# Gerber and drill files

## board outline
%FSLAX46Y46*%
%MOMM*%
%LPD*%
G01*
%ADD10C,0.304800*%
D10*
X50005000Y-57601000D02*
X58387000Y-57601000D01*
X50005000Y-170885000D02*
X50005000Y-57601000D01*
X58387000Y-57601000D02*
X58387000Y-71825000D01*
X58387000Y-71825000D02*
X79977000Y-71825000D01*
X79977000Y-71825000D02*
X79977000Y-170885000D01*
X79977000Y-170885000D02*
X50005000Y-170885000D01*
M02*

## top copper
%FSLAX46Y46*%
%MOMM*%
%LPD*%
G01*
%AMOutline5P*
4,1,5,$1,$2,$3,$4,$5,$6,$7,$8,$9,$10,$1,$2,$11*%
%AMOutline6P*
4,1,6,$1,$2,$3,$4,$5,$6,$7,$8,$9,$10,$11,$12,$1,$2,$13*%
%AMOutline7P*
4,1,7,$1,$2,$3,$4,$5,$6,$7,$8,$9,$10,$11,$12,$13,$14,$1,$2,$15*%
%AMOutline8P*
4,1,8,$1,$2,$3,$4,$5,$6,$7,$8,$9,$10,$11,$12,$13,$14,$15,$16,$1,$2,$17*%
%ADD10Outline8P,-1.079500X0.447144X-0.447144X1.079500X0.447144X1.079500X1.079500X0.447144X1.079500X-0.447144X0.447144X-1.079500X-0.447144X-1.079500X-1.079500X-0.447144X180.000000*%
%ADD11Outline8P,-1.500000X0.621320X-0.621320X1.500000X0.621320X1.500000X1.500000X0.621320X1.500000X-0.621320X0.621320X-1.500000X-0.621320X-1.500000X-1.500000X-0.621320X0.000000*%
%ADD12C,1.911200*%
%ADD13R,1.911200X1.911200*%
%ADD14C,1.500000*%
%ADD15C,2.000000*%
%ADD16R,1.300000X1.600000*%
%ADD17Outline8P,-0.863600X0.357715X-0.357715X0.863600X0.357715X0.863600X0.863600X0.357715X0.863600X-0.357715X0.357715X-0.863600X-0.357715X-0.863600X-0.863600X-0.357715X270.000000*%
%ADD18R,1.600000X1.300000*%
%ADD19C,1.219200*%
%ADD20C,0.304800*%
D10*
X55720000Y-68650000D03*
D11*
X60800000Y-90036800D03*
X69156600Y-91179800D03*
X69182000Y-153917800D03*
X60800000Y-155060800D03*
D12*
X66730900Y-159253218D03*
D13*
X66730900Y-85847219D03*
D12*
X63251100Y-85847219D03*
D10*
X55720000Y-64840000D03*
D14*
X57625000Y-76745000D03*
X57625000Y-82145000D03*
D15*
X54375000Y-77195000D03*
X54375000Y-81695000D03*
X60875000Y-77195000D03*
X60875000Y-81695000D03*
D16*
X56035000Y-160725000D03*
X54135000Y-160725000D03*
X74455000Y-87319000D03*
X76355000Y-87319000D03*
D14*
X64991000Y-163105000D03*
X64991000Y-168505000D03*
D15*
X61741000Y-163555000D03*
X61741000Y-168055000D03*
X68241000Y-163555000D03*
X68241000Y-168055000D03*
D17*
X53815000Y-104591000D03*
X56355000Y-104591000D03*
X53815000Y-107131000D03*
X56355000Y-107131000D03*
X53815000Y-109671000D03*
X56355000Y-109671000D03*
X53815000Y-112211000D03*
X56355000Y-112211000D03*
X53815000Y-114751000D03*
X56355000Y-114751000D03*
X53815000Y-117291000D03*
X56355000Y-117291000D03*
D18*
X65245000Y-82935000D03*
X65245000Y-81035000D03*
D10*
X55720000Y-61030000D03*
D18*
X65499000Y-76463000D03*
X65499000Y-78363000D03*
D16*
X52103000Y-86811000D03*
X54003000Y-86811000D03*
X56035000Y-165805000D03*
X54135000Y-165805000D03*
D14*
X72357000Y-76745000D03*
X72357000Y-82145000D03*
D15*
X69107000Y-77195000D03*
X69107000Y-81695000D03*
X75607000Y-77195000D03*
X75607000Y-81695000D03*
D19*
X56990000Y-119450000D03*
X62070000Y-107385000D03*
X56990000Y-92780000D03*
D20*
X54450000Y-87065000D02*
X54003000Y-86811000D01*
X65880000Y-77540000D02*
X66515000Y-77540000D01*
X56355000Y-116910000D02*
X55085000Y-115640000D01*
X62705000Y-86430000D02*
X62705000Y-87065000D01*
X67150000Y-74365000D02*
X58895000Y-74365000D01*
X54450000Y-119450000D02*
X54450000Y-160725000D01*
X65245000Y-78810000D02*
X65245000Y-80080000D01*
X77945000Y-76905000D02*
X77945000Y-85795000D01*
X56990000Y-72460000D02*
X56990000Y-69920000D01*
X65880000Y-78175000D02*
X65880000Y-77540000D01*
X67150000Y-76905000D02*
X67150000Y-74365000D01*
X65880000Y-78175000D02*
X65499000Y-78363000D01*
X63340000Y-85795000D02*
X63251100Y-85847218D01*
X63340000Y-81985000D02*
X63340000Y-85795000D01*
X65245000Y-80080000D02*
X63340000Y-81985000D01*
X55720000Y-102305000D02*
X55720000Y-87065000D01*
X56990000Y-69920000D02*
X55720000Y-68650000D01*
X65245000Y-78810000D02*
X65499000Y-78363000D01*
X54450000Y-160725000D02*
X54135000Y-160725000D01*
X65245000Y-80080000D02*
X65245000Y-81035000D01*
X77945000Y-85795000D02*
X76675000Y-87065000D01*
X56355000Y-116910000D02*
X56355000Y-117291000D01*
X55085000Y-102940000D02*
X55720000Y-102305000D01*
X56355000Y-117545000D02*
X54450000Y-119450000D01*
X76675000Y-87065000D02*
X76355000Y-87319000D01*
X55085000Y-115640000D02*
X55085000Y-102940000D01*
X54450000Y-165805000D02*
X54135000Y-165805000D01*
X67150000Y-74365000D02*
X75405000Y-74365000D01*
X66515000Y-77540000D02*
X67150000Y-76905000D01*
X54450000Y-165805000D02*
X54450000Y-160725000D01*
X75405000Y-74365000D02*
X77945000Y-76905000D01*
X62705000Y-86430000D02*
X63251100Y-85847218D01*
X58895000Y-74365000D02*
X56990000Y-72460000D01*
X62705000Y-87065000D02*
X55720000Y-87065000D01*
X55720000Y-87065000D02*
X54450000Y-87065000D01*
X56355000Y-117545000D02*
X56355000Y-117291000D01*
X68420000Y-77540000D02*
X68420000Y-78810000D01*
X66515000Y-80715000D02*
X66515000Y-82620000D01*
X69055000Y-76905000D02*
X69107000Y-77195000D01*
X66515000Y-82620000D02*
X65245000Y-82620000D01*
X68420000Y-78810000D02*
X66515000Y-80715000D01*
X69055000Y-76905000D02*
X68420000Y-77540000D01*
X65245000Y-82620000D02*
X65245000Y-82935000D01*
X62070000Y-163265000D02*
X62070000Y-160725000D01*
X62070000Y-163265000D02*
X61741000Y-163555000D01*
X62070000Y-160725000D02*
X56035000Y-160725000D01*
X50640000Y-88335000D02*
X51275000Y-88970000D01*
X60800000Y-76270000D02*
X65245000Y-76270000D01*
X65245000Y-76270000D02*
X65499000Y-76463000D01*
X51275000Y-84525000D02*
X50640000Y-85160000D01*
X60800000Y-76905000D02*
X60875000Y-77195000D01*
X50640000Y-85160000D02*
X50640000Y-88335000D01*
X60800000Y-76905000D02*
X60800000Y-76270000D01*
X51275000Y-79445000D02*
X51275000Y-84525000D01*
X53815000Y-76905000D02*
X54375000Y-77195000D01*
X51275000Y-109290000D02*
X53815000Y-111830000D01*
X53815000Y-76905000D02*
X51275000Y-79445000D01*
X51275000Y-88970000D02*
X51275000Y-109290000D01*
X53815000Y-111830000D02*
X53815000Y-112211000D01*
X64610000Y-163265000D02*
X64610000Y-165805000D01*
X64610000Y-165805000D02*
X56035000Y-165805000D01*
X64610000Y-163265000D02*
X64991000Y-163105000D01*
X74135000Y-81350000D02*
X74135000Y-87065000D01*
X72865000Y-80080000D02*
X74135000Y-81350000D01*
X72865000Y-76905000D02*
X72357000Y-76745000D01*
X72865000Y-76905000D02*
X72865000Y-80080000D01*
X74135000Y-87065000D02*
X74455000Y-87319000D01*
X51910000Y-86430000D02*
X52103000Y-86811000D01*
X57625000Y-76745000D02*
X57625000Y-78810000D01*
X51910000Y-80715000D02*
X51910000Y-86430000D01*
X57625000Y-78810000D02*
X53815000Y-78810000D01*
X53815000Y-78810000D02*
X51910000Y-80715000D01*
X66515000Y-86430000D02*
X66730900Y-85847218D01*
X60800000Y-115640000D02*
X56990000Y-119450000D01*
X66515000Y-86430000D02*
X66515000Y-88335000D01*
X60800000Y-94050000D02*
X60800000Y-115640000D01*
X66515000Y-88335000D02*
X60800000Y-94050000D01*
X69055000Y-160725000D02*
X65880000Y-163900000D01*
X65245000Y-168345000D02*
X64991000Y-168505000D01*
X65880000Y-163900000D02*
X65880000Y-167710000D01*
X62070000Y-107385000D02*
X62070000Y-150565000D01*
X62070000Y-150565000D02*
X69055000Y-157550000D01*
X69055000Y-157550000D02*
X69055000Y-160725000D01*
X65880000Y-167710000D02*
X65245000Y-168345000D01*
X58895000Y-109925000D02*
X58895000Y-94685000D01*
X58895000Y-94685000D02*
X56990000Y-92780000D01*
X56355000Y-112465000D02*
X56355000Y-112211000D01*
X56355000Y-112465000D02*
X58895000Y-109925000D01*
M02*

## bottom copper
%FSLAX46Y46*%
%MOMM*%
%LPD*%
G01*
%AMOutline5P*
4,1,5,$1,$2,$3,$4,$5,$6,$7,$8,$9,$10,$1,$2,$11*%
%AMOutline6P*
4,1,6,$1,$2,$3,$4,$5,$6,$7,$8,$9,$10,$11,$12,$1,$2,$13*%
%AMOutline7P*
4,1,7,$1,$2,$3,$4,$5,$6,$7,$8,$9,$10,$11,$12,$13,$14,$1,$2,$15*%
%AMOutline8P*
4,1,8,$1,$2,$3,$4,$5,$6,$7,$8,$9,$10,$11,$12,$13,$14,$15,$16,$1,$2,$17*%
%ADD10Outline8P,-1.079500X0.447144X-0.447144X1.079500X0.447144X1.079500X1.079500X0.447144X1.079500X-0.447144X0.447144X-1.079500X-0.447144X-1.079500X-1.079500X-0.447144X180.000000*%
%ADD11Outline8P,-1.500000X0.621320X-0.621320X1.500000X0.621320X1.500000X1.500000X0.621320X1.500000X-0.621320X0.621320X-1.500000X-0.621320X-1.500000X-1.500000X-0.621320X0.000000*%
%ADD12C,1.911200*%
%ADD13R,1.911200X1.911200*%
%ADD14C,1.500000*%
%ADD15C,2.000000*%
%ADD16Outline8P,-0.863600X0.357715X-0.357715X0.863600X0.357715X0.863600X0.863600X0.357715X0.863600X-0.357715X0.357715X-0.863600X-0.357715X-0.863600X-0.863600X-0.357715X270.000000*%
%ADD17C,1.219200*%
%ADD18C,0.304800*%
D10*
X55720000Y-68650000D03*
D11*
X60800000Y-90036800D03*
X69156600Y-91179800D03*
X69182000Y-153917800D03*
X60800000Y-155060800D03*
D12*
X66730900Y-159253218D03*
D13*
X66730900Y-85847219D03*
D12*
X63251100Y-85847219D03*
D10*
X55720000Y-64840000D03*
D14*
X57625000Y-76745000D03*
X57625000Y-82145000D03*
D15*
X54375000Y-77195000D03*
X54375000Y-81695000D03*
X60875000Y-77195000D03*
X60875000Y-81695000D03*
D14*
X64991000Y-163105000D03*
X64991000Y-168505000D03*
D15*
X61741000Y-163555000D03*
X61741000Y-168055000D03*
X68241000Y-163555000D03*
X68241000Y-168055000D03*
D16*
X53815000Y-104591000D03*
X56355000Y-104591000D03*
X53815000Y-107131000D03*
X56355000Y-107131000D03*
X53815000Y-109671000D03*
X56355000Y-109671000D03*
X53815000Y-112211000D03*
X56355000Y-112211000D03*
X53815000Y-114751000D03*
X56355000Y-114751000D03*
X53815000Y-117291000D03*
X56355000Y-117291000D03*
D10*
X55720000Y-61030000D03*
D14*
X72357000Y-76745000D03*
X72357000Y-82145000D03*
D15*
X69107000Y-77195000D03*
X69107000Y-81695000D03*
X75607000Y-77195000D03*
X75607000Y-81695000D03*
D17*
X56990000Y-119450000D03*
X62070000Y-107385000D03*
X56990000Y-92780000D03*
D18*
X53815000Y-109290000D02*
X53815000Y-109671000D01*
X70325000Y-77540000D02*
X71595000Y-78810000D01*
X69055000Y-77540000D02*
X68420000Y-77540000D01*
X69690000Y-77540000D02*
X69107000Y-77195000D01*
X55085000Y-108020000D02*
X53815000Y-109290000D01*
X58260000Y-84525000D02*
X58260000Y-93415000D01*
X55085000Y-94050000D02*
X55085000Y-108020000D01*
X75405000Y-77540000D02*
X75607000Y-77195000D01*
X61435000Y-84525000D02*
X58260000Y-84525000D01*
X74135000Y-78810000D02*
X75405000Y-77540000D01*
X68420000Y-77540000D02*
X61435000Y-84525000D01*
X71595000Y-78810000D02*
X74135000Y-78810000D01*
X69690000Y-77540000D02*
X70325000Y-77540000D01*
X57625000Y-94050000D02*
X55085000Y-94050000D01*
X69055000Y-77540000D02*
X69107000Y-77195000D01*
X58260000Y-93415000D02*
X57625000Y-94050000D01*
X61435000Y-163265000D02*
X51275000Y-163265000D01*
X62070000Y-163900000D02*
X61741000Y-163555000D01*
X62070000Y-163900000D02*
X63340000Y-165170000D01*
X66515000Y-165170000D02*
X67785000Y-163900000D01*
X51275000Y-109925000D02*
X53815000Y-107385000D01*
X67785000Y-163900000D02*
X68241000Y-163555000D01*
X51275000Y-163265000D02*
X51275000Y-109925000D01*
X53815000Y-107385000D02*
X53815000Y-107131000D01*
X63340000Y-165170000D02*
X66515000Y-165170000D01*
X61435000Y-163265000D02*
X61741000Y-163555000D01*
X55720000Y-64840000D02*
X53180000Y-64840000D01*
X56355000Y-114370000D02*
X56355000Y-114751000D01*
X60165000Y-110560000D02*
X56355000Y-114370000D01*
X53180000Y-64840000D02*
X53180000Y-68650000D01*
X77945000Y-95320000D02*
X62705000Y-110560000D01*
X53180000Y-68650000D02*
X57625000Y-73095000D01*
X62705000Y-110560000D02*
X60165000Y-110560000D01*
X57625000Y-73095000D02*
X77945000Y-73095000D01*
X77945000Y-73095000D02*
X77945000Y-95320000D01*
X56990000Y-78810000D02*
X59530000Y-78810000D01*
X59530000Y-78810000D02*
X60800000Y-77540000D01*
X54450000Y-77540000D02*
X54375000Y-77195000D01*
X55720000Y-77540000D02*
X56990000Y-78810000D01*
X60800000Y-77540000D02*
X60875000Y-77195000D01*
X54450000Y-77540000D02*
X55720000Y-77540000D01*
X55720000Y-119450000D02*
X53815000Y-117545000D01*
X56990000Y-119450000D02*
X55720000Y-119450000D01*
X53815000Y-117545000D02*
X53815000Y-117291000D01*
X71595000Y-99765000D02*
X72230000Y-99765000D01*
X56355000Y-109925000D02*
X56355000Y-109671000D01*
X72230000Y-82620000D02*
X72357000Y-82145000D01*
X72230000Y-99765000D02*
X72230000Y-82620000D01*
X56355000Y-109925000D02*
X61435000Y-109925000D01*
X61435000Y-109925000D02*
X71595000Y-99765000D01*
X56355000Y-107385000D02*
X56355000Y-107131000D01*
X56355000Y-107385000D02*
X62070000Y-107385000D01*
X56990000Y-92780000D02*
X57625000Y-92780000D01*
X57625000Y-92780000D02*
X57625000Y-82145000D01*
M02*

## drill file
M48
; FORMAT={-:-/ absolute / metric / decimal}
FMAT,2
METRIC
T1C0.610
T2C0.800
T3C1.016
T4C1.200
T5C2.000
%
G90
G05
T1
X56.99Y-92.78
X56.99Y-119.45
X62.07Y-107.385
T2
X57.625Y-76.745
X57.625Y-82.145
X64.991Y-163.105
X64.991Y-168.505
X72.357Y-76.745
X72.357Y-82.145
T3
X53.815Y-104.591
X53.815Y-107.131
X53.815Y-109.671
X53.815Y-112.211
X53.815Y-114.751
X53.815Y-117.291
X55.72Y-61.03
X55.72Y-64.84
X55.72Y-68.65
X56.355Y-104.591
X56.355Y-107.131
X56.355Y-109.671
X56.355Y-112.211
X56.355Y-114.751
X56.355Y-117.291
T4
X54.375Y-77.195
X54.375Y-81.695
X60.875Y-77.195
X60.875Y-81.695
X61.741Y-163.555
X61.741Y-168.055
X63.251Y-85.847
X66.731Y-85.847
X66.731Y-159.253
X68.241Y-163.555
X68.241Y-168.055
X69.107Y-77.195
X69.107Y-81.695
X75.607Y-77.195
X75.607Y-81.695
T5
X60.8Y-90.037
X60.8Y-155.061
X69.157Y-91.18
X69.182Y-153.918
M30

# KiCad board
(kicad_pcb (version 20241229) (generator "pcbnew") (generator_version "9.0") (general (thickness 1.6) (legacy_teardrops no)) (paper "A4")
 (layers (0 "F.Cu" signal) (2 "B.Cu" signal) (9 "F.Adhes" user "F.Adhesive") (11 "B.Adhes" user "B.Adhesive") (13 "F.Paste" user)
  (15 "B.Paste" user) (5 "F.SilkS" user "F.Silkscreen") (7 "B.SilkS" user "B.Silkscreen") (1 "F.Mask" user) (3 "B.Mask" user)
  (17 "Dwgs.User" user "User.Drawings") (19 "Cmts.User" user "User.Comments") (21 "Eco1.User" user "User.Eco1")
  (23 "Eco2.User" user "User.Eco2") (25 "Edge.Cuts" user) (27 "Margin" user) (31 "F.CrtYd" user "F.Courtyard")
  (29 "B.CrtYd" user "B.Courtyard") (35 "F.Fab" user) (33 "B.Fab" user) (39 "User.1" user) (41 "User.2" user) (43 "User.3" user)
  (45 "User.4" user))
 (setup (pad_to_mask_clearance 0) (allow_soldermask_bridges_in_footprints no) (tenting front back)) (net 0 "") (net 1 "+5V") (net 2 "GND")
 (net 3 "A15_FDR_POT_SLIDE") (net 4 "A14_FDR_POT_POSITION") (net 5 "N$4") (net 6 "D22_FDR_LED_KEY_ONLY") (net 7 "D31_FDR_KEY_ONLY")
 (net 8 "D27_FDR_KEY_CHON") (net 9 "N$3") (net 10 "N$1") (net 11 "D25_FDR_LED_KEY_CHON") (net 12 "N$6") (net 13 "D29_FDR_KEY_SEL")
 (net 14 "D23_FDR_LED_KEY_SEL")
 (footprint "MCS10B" (layer "F.Cu") (at 55.72 68.65 180)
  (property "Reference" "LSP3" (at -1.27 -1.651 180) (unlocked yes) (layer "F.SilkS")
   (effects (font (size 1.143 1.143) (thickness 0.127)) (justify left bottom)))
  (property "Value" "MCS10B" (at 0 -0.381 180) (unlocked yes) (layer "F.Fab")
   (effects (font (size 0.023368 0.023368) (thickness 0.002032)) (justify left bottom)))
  (pad "MP" thru_hole roundrect (at 0 0 180) (size 2.159 2.159) (drill 1.016) (layers "*.Cu" "*.Mask") (remove_unused_layers no)
   (roundrect_rratio 0.25) (chamfer_ratio 0.2928932188) (chamfer top_left top_right bottom_left bottom_right) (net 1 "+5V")
   (solder_mask_margin 0.1016) (thermal_bridge_angle 0)))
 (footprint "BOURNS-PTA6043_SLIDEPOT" (layer "F.Cu") (at 64.991 116.529)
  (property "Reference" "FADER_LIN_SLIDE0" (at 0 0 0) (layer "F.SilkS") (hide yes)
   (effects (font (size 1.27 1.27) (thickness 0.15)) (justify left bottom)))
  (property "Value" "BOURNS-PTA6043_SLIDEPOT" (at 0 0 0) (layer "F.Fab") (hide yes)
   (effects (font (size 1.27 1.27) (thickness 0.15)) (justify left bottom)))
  (pad "MOUNT1" thru_hole roundrect (at -4.191 -26.4922) (size 3 3) (drill 2) (layers "*.Cu" "*.Mask") (remove_unused_layers no)
   (roundrect_rratio 0.25) (chamfer_ratio 0.2928932188) (chamfer top_left top_right bottom_left bottom_right) (solder_mask_margin 0.1016)
   (thermal_bridge_angle 0))
  (pad "MOUNT2" thru_hole roundrect (at 4.1656 -25.3492) (size 3 3) (drill 2) (layers "*.Cu" "*.Mask") (remove_unused_layers no)
   (roundrect_rratio 0.25) (chamfer_ratio 0.2928932188) (chamfer top_left top_right bottom_left bottom_right) (solder_mask_margin 0.1016)
   (thermal_bridge_angle 0))
  (pad "MOUNT3" thru_hole roundrect (at 4.191 37.3888) (size 3 3) (drill 2) (layers "*.Cu" "*.Mask") (remove_unused_layers no)
   (roundrect_rratio 0.25) (chamfer_ratio 0.2928932188) (chamfer top_left top_right bottom_left bottom_right) (solder_mask_margin 0.1016)
   (thermal_bridge_angle 0))
  (pad "MOUNT4" thru_hole roundrect (at -4.191 38.5318) (size 3 3) (drill 2) (layers "*.Cu" "*.Mask") (remove_unused_layers no)
   (roundrect_rratio 0.25) (chamfer_ratio 0.2928932188) (chamfer top_left top_right bottom_left bottom_right) (solder_mask_margin 0.1016)
   (thermal_bridge_angle 0))
  (pad "P$1" thru_hole circle (at 1.7399 42.724218) (size 1.9112 1.9112) (drill 1.2) (layers "*.Cu" "*.Mask") (remove_unused_layers no)
   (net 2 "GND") (solder_mask_margin 0.1016) (thermal_bridge_angle 0))
  (pad "P$2" thru_hole rect (at 1.7399 -30.681781) (size 1.9112 1.9112) (drill 1.2) (layers "*.Cu" "*.Mask") (remove_unused_layers no)
   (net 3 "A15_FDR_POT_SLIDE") (solder_mask_margin 0.1016) (thermal_bridge_angle 0))
  (pad "P$3" thru_hole circle (at -1.7399 -30.681781) (size 1.9112 1.9112) (drill 1.2) (layers "*.Cu" "*.Mask") (remove_unused_layers no)
   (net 1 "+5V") (solder_mask_margin 0.1016) (thermal_bridge_angle 0)))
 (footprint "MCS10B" (layer "F.Cu") (at 55.72 64.84 180)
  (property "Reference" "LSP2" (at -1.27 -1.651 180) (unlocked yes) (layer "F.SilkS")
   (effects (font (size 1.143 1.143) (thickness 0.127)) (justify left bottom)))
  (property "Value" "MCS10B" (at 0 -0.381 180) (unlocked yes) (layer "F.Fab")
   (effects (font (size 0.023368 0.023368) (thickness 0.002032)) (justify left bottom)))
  (pad "MP" thru_hole roundrect (at 0 0 180) (size 2.159 2.159) (drill 1.016) (layers "*.Cu" "*.Mask") (remove_unused_layers no)
   (roundrect_rratio 0.25) (chamfer_ratio 0.2928932188) (chamfer top_left top_right bottom_left bottom_right) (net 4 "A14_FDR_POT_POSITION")
   (solder_mask_margin 0.1016) (thermal_bridge_angle 0)))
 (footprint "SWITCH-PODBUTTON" (layer "F.Cu") (at 57.625 79.445)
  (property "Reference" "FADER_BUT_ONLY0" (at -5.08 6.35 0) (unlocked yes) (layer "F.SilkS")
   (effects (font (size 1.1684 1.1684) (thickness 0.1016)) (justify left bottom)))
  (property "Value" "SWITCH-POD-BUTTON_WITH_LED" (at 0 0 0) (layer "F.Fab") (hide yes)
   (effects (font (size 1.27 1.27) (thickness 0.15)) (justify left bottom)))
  (pad "LEDA" thru_hole circle (at 0 -2.7) (size 1.5 1.5) (drill 0.8) (layers "*.Cu" "*.Mask") (remove_unused_layers no) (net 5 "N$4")
   (solder_mask_margin 0.1016) (thermal_bridge_angle 0))
  (pad "LEDB" thru_hole circle (at 0 2.7) (size 1.5 1.5) (drill 0.8) (layers "*.Cu" "*.Mask") (remove_unused_layers no)
   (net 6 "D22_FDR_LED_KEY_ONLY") (solder_mask_margin 0.1016) (thermal_bridge_angle 0))
  (pad "SW1A" thru_hole circle (at -3.25 -2.25) (size 2 2) (drill 1.2) (layers "*.Cu" "*.Mask") (remove_unused_layers no)
   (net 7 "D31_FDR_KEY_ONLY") (solder_mask_margin 0.1016) (thermal_bridge_angle 0))
  (pad "SW1B" thru_hole circle (at -3.25 2.25) (size 2 2) (drill 1.2) (layers "*.Cu" "*.Mask") (remove_unused_layers no) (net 2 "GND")
   (solder_mask_margin 0.1016) (thermal_bridge_angle 0))
  (pad "SW2A" thru_hole circle (at 3.25 -2.25) (size 2 2) (drill 1.2) (layers "*.Cu" "*.Mask") (remove_unused_layers no)
   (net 7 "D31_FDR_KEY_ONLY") (solder_mask_margin 0.1016) (thermal_bridge_angle 0))
  (pad "SW2B" thru_hole circle (at 3.25 2.25) (size 2 2) (drill 1.2) (layers "*.Cu" "*.Mask") (remove_unused_layers no) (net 2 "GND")
   (solder_mask_margin 0.1016) (thermal_bridge_angle 0)))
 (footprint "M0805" (layer "F.Cu") (at 55.085 160.725 180)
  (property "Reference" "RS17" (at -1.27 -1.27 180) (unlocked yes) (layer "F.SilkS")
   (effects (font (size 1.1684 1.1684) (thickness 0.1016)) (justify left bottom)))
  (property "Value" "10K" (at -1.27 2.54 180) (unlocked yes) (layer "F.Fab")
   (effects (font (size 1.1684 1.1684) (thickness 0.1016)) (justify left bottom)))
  (pad "1" smd rect (at -0.95 0 180) (size 1.3 1.6) (layers "F.Cu" "F.Mask" "F.Paste") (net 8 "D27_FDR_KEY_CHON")
   (solder_mask_margin 0.1016) (solder_paste_margin 0) (thermal_bridge_angle 0))
  (pad "2" smd rect (at 0.95 0 180) (size 1.3 1.6) (layers "F.Cu" "F.Mask" "F.Paste") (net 1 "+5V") (solder_mask_margin 0.1016)
   (solder_paste_margin 0) (thermal_bridge_angle 0)))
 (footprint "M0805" (layer "F.Cu") (at 75.405 87.319)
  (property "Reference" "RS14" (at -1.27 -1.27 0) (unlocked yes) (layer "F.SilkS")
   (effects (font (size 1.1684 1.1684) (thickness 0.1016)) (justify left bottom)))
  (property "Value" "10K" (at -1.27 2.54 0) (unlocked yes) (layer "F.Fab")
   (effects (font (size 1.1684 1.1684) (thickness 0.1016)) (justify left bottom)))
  (pad "1" smd rect (at -0.95 0) (size 1.3 1.6) (layers "F.Cu" "F.Mask" "F.Paste") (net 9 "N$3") (solder_mask_margin 0.1016)
   (solder_paste_margin 0) (thermal_bridge_angle 0))
  (pad "2" smd rect (at 0.95 0) (size 1.3 1.6) (layers "F.Cu" "F.Mask" "F.Paste") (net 1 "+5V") (solder_mask_margin 0.1016)
   (solder_paste_margin 0) (thermal_bridge_angle 0)))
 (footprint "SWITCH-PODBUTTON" (layer "F.Cu") (at 64.991 165.805)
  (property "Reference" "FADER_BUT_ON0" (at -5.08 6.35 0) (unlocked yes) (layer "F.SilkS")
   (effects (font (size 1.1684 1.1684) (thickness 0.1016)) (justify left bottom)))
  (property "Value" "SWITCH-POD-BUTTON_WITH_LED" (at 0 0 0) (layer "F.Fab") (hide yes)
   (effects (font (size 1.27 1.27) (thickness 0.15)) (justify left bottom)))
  (pad "LEDA" thru_hole circle (at 0 -2.7) (size 1.5 1.5) (drill 0.8) (layers "*.Cu" "*.Mask") (remove_unused_layers no) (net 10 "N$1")
   (solder_mask_margin 0.1016) (thermal_bridge_angle 0))
  (pad "LEDB" thru_hole circle (at 0 2.7) (size 1.5 1.5) (drill 0.8) (layers "*.Cu" "*.Mask") (remove_unused_layers no)
   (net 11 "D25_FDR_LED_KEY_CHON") (solder_mask_margin 0.1016) (thermal_bridge_angle 0))
  (pad "SW1A" thru_hole circle (at -3.25 -2.25) (size 2 2) (drill 1.2) (layers "*.Cu" "*.Mask") (remove_unused_layers no)
   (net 8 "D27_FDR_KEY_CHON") (solder_mask_margin 0.1016) (thermal_bridge_angle 0))
  (pad "SW1B" thru_hole circle (at -3.25 2.25) (size 2 2) (drill 1.2) (layers "*.Cu" "*.Mask") (remove_unused_layers no) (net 2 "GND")
   (solder_mask_margin 0.1016) (thermal_bridge_angle 0))
  (pad "SW2A" thru_hole circle (at 3.25 -2.25) (size 2 2) (drill 1.2) (layers "*.Cu" "*.Mask") (remove_unused_layers no)
   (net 8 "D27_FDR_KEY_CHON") (solder_mask_margin 0.1016) (thermal_bridge_angle 0))
  (pad "SW2B" thru_hole circle (at 3.25 2.25) (size 2 2) (drill 1.2) (layers "*.Cu" "*.Mask") (remove_unused_layers no) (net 2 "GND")
   (solder_mask_margin 0.1016) (thermal_bridge_angle 0)))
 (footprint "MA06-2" (layer "F.Cu") (at 55.085 110.941 -90)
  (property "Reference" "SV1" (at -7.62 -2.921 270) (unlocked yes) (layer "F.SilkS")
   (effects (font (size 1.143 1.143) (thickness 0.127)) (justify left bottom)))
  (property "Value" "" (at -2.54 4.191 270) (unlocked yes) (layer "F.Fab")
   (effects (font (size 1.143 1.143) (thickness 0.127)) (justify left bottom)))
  (pad "1" thru_hole roundrect (at -6.35 1.27 270) (size 1.7272 1.7272) (drill 1.016) (layers "*.Cu" "*.Mask") (remove_unused_layers no)
   (roundrect_rratio 0.25) (chamfer_ratio 0.2928932188) (chamfer top_left top_right bottom_left bottom_right) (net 2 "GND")
   (solder_mask_margin 0.1016) (thermal_bridge_angle 0))
  (pad "2" thru_hole roundrect (at -6.35 -1.27 270) (size 1.7272 1.7272) (drill 1.016) (layers "*.Cu" "*.Mask") (remove_unused_layers no)
   (roundrect_rratio 0.25) (chamfer_ratio 0.2928932188) (chamfer top_left top_right bottom_left bottom_right) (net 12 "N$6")
   (solder_mask_margin 0.1016) (thermal_bridge_angle 0))
  (pad "3" thru_hole roundrect (at -3.81 1.27 270) (size 1.7272 1.7272) (drill 1.016) (layers "*.Cu" "*.Mask") (remove_unused_layers no)
   (roundrect_rratio 0.25) (chamfer_ratio 0.2928932188) (chamfer top_left top_right bottom_left bottom_right) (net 8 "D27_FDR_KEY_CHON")
   (solder_mask_margin 0.1016) (thermal_bridge_angle 0))
  (pad "4" thru_hole roundrect (at -3.81 -1.27 270) (size 1.7272 1.7272) (drill 1.016) (layers "*.Cu" "*.Mask") (remove_unused_layers no)
   (roundrect_rratio 0.25) (chamfer_ratio 0.2928932188) (chamfer top_left top_right bottom_left bottom_right)
   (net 11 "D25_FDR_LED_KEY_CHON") (solder_mask_margin 0.1016) (thermal_bridge_angle 0))
  (pad "5" thru_hole roundrect (at -1.27 1.27 270) (size 1.7272 1.7272) (drill 1.016) (layers "*.Cu" "*.Mask") (remove_unused_layers no)
   (roundrect_rratio 0.25) (chamfer_ratio 0.2928932188) (chamfer top_left top_right bottom_left bottom_right) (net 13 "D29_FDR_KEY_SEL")
   (solder_mask_margin 0.1016) (thermal_bridge_angle 0))
  (pad "6" thru_hole roundrect (at -1.27 -1.27 270) (size 1.7272 1.7272) (drill 1.016) (layers "*.Cu" "*.Mask") (remove_unused_layers no)
   (roundrect_rratio 0.25) (chamfer_ratio 0.2928932188) (chamfer top_left top_right bottom_left bottom_right) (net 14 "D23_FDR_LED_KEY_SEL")
   (solder_mask_margin 0.1016) (thermal_bridge_angle 0))
  (pad "7" thru_hole roundrect (at 1.27 1.27 270) (size 1.7272 1.7272) (drill 1.016) (layers "*.Cu" "*.Mask") (remove_unused_layers no)
   (roundrect_rratio 0.25) (chamfer_ratio 0.2928932188) (chamfer top_left top_right bottom_left bottom_right) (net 7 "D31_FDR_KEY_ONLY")
   (solder_mask_margin 0.1016) (thermal_bridge_angle 0))
  (pad "8" thru_hole roundrect (at 1.27 -1.27 270) (size 1.7272 1.7272) (drill 1.016) (layers "*.Cu" "*.Mask") (remove_unused_layers no)
   (roundrect_rratio 0.25) (chamfer_ratio 0.2928932188) (chamfer top_left top_right bottom_left bottom_right) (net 6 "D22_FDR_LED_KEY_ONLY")
   (solder_mask_margin 0.1016) (thermal_bridge_angle 0))
  (pad "9" thru_hole roundrect (at 3.81 1.27 270) (size 1.7272 1.7272) (drill 1.016) (layers "*.Cu" "*.Mask") (remove_unused_layers no)
   (roundrect_rratio 0.25) (chamfer_ratio 0.2928932188) (chamfer top_left top_right bottom_left bottom_right) (solder_mask_margin 0.1016)
   (thermal_bridge_angle 0))
  (pad "10" thru_hole roundrect (at 3.81 -1.27 270) (size 1.7272 1.7272) (drill 1.016) (layers "*.Cu" "*.Mask") (remove_unused_layers no)
   (roundrect_rratio 0.25) (chamfer_ratio 0.2928932188) (chamfer top_left top_right bottom_left bottom_right) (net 4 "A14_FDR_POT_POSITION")
   (solder_mask_margin 0.1016) (thermal_bridge_angle 0))
  (pad "11" thru_hole roundrect (at 6.35 1.27 270) (size 1.7272 1.7272) (drill 1.016) (layers "*.Cu" "*.Mask") (remove_unused_layers no)
   (roundrect_rratio 0.25) (chamfer_ratio 0.2928932188) (chamfer top_left top_right bottom_left bottom_right) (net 3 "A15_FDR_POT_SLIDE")
   (solder_mask_margin 0.1016) (thermal_bridge_angle 0))
  (pad "12" thru_hole roundrect (at 6.35 -1.27 270) (size 1.7272 1.7272) (drill 1.016) (layers "*.Cu" "*.Mask") (remove_unused_layers no)
   (roundrect_rratio 0.25) (chamfer_ratio 0.2928932188) (chamfer top_left top_right bottom_left bottom_right) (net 1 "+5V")
   (solder_mask_margin 0.1016) (thermal_bridge_angle 0)))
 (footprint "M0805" (layer "F.Cu") (at 65.245 81.985 90)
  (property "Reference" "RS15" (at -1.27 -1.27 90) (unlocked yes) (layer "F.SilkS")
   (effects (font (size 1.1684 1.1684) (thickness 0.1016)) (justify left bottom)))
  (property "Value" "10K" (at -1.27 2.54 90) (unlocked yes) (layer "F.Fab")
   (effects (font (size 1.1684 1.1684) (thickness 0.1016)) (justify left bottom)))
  (pad "1" smd rect (at -0.95 0 90) (size 1.3 1.6) (layers "F.Cu" "F.Mask" "F.Paste") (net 13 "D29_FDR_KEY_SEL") (solder_mask_margin 0.1016)
   (solder_paste_margin 0) (thermal_bridge_angle 0))
  (pad "2" smd rect (at 0.95 0 90) (size 1.3 1.6) (layers "F.Cu" "F.Mask" "F.Paste") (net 1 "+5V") (solder_mask_margin 0.1016)
   (solder_paste_margin 0) (thermal_bridge_angle 0)))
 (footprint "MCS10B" (layer "F.Cu") (at 55.72 61.03 180)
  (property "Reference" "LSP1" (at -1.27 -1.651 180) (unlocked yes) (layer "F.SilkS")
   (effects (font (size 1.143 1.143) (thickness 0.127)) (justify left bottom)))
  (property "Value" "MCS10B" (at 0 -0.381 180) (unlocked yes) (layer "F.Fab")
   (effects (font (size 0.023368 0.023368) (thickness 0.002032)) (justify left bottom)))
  (pad "MP" thru_hole roundrect (at 0 0 180) (size 2.159 2.159) (drill 1.016) (layers "*.Cu" "*.Mask") (remove_unused_layers no)
   (roundrect_rratio 0.25) (chamfer_ratio 0.2928932188) (chamfer top_left top_right bottom_left bottom_right) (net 2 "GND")
   (solder_mask_margin 0.1016) (thermal_bridge_angle 0)))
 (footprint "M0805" (layer "F.Cu") (at 65.499 77.413 -90)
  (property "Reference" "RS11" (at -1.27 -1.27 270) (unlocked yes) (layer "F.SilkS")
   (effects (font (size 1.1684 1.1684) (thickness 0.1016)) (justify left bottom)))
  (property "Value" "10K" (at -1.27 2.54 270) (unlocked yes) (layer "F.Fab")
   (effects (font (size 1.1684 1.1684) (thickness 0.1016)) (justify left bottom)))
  (pad "1" smd rect (at -0.95 0 270) (size 1.3 1.6) (layers "F.Cu" "F.Mask" "F.Paste") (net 7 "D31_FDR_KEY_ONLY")
   (solder_mask_margin 0.1016) (solder_paste_margin 0) (thermal_bridge_angle 0))
  (pad "2" smd rect (at 0.95 0 270) (size 1.3 1.6) (layers "F.Cu" "F.Mask" "F.Paste") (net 1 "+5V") (solder_mask_margin 0.1016)
   (solder_paste_margin 0) (thermal_bridge_angle 0)))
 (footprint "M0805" (layer "F.Cu") (at 53.053 86.811)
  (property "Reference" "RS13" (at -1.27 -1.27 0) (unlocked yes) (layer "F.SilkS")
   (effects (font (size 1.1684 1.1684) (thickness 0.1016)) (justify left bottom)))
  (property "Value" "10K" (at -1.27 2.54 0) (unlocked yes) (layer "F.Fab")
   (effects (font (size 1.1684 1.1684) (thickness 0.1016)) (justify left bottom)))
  (pad "1" smd rect (at -0.95 0) (size 1.3 1.6) (layers "F.Cu" "F.Mask" "F.Paste") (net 5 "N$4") (solder_mask_margin 0.1016)
   (solder_paste_margin 0) (thermal_bridge_angle 0))
  (pad "2" smd rect (at 0.95 0) (size 1.3 1.6) (layers "F.Cu" "F.Mask" "F.Paste") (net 1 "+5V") (solder_mask_margin 0.1016)
   (solder_paste_margin 0) (thermal_bridge_angle 0)))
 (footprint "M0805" (layer "F.Cu") (at 55.085 165.805 180)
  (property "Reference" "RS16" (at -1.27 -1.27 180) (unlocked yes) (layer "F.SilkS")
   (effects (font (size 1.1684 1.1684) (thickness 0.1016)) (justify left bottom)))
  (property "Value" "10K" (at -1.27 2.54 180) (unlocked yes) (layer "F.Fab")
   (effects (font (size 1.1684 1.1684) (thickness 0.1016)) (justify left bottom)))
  (pad "1" smd rect (at -0.95 0 180) (size 1.3 1.6) (layers "F.Cu" "F.Mask" "F.Paste") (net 10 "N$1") (solder_mask_margin 0.1016)
   (solder_paste_margin 0) (thermal_bridge_angle 0))
  (pad "2" smd rect (at 0.95 0 180) (size 1.3 1.6) (layers "F.Cu" "F.Mask" "F.Paste") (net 1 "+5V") (solder_mask_margin 0.1016)
   (solder_paste_margin 0) (thermal_bridge_angle 0)))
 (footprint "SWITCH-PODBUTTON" (layer "F.Cu") (at 72.357 79.445)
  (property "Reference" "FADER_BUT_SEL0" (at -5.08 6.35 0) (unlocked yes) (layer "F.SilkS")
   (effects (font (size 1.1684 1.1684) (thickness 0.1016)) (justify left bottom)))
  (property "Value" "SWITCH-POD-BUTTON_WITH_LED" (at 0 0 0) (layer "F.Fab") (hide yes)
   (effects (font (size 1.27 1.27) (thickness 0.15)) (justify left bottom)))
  (pad "LEDA" thru_hole circle (at 0 -2.7) (size 1.5 1.5) (drill 0.8) (layers "*.Cu" "*.Mask") (remove_unused_layers no) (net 9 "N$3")
   (solder_mask_margin 0.1016) (thermal_bridge_angle 0))
  (pad "LEDB" thru_hole circle (at 0 2.7) (size 1.5 1.5) (drill 0.8) (layers "*.Cu" "*.Mask") (remove_unused_layers no)
   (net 14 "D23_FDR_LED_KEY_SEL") (solder_mask_margin 0.1016) (thermal_bridge_angle 0))
  (pad "SW1A" thru_hole circle (at -3.25 -2.25) (size 2 2) (drill 1.2) (layers "*.Cu" "*.Mask") (remove_unused_layers no)
   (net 13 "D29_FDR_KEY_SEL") (solder_mask_margin 0.1016) (thermal_bridge_angle 0))
  (pad "SW1B" thru_hole circle (at -3.25 2.25) (size 2 2) (drill 1.2) (layers "*.Cu" "*.Mask") (remove_unused_layers no) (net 2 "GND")
   (solder_mask_margin 0.1016) (thermal_bridge_angle 0))
  (pad "SW2A" thru_hole circle (at 3.25 -2.25) (size 2 2) (drill 1.2) (layers "*.Cu" "*.Mask") (remove_unused_layers no)
   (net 13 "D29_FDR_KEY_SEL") (solder_mask_margin 0.1016) (thermal_bridge_angle 0))
  (pad "SW2B" thru_hole circle (at 3.25 2.25) (size 2 2) (drill 1.2) (layers "*.Cu" "*.Mask") (remove_unused_layers no) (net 2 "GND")
   (solder_mask_margin 0.1016) (thermal_bridge_angle 0)))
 (gr_line (start 50.005 57.601) (end 58.387 57.601) (stroke (width 0.3048) (type solid)) (layer "Edge.Cuts"))
 (gr_line (start 50.005 170.885) (end 50.005 57.601) (stroke (width 0.3048) (type solid)) (layer "Edge.Cuts"))
 (gr_line (start 58.387 57.601) (end 58.387 71.825) (stroke (width 0.3048) (type solid)) (layer "Edge.Cuts"))
 (gr_line (start 58.387 71.825) (end 79.977 71.825) (stroke (width 0.3048) (type solid)) (layer "Edge.Cuts"))
 (gr_line (start 79.977 71.825) (end 79.977 170.885) (stroke (width 0.3048) (type solid)) (layer "Edge.Cuts"))
 (gr_line (start 79.977 170.885) (end 50.005 170.885) (stroke (width 0.3048) (type solid)) (layer "Edge.Cuts"))
 (segment (start 54.45 87.065) (end 54.003 86.811) (width 0.3048) (layer "F.Cu") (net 1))
 (segment (start 65.88 77.54) (end 66.515 77.54) (width 0.3048) (layer "F.Cu") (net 1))
 (segment (start 56.355 116.91) (end 55.085 115.64) (width 0.3048) (layer "F.Cu") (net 1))
 (segment (start 62.705 86.43) (end 62.705 87.065) (width 0.3048) (layer "F.Cu") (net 1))
 (segment (start 67.15 74.365) (end 58.895 74.365) (width 0.3048) (layer "F.Cu") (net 1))
 (segment (start 54.45 119.45) (end 54.45 160.725) (width 0.3048) (layer "F.Cu") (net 1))
 (segment (start 65.245 78.81) (end 65.245 80.08) (width 0.3048) (layer "F.Cu") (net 1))
 (segment (start 77.945 76.905) (end 77.945 85.795) (width 0.3048) (layer "F.Cu") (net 1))
 (segment (start 56.99 72.46) (end 56.99 69.92) (width 0.3048) (layer "F.Cu") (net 1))
 (segment (start 65.88 78.175) (end 65.88 77.54) (width 0.3048) (layer "F.Cu") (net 1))
 (segment (start 67.15 76.905) (end 67.15 74.365) (width 0.3048) (layer "F.Cu") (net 1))
 (segment (start 65.88 78.175) (end 65.499 78.363) (width 0.3048) (layer "F.Cu") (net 1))
 (segment (start 63.34 85.795) (end 63.2511 85.847218) (width 0.3048) (layer "F.Cu") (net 1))
 (segment (start 63.34 81.985) (end 63.34 85.795) (width 0.3048) (layer "F.Cu") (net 1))
 (segment (start 65.245 80.08) (end 63.34 81.985) (width 0.3048) (layer "F.Cu") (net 1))
 (segment (start 55.72 102.305) (end 55.72 87.065) (width 0.3048) (layer "F.Cu") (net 1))
 (segment (start 56.99 69.92) (end 55.72 68.65) (width 0.3048) (layer "F.Cu") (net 1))
 (segment (start 65.245 78.81) (end 65.499 78.363) (width 0.3048) (layer "F.Cu") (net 1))
 (segment (start 54.45 160.725) (end 54.135 160.725) (width 0.3048) (layer "F.Cu") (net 1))
 (segment (start 65.245 80.08) (end 65.245 81.035) (width 0.3048) (layer "F.Cu") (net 1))
 (segment (start 77.945 85.795) (end 76.675 87.065) (width 0.3048) (layer "F.Cu") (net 1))
 (segment (start 56.355 116.91) (end 56.355 117.291) (width 0.3048) (layer "F.Cu") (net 1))
 (segment (start 55.085 102.94) (end 55.72 102.305) (width 0.3048) (layer "F.Cu") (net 1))
 (segment (start 56.355 117.545) (end 54.45 119.45) (width 0.3048) (layer "F.Cu") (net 1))
 (segment (start 76.675 87.065) (end 76.355 87.319) (width 0.3048) (layer "F.Cu") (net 1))
 (segment (start 55.085 115.64) (end 55.085 102.94) (width 0.3048) (layer "F.Cu") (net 1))
 (segment (start 54.45 165.805) (end 54.135 165.805) (width 0.3048) (layer "F.Cu") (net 1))
 (segment (start 67.15 74.365) (end 75.405 74.365) (width 0.3048) (layer "F.Cu") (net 1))
 (segment (start 66.515 77.54) (end 67.15 76.905) (width 0.3048) (layer "F.Cu") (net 1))
 (segment (start 54.45 165.805) (end 54.45 160.725) (width 0.3048) (layer "F.Cu") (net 1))
 (segment (start 75.405 74.365) (end 77.945 76.905) (width 0.3048) (layer "F.Cu") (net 1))
 (segment (start 62.705 86.43) (end 63.2511 85.847218) (width 0.3048) (layer "F.Cu") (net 1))
 (segment (start 58.895 74.365) (end 56.99 72.46) (width 0.3048) (layer "F.Cu") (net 1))
 (segment (start 62.705 87.065) (end 55.72 87.065) (width 0.3048) (layer "F.Cu") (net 1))
 (segment (start 55.72 87.065) (end 54.45 87.065) (width 0.3048) (layer "F.Cu") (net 1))
 (segment (start 56.355 117.545) (end 56.355 117.291) (width 0.3048) (layer "F.Cu") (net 1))
 (segment (start 68.42 77.54) (end 68.42 78.81) (width 0.3048) (layer "F.Cu") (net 13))
 (segment (start 66.515 80.715) (end 66.515 82.62) (width 0.3048) (layer "F.Cu") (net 13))
 (segment (start 69.055 76.905) (end 69.107 77.195) (width 0.3048) (layer "F.Cu") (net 13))
 (segment (start 66.515 82.62) (end 65.245 82.62) (width 0.3048) (layer "F.Cu") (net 13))
 (segment (start 68.42 78.81) (end 66.515 80.715) (width 0.3048) (layer "F.Cu") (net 13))
 (segment (start 69.055 76.905) (end 68.42 77.54) (width 0.3048) (layer "F.Cu") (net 13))
 (segment (start 65.245 82.62) (end 65.245 82.935) (width 0.3048) (layer "F.Cu") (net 13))
 (segment (start 53.815 109.29) (end 53.815 109.671) (width 0.3048) (layer "B.Cu") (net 13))
 (segment (start 70.325 77.54) (end 71.595 78.81) (width 0.3048) (layer "B.Cu") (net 13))
 (segment (start 69.055 77.54) (end 68.42 77.54) (width 0.3048) (layer "B.Cu") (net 13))
 (segment (start 69.69 77.54) (end 69.107 77.195) (width 0.3048) (layer "B.Cu") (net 13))
 (segment (start 55.085 108.02) (end 53.815 109.29) (width 0.3048) (layer "B.Cu") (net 13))
 (segment (start 58.26 84.525) (end 58.26 93.415) (width 0.3048) (layer "B.Cu") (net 13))
 (segment (start 55.085 94.05) (end 55.085 108.02) (width 0.3048) (layer "B.Cu") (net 13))
 (segment (start 75.405 77.54) (end 75.607 77.195) (width 0.3048) (layer "B.Cu") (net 13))
 (segment (start 61.435 84.525) (end 58.26 84.525) (width 0.3048) (layer "B.Cu") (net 13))
 (segment (start 74.135 78.81) (end 75.405 77.54) (width 0.3048) (layer "B.Cu") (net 13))
 (segment (start 68.42 77.54) (end 61.435 84.525) (width 0.3048) (layer "B.Cu") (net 13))
 (segment (start 71.595 78.81) (end 74.135 78.81) (width 0.3048) (layer "B.Cu") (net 13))
 (segment (start 69.69 77.54) (end 70.325 77.54) (width 0.3048) (layer "B.Cu") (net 13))
 (segment (start 57.625 94.05) (end 55.085 94.05) (width 0.3048) (layer "B.Cu") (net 13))
 (segment (start 69.055 77.54) (end 69.107 77.195) (width 0.3048) (layer "B.Cu") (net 13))
 (segment (start 58.26 93.415) (end 57.625 94.05) (width 0.3048) (layer "B.Cu") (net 13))
 (segment (start 62.07 163.265) (end 62.07 160.725) (width 0.3048) (layer "F.Cu") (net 8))
 (segment (start 62.07 163.265) (end 61.741 163.555) (width 0.3048) (layer "F.Cu") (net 8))
 (segment (start 62.07 160.725) (end 56.035 160.725) (width 0.3048) (layer "F.Cu") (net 8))
 (segment (start 61.435 163.265) (end 51.275 163.265) (width 0.3048) (layer "B.Cu") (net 8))
 (segment (start 62.07 163.9) (end 61.741 163.555) (width 0.3048) (layer "B.Cu") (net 8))
 (segment (start 62.07 163.9) (end 63.34 165.17) (width 0.3048) (layer "B.Cu") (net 8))
 (segment (start 66.515 165.17) (end 67.785 163.9) (width 0.3048) (layer "B.Cu") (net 8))
 (segment (start 51.275 109.925) (end 53.815 107.385) (width 0.3048) (layer "B.Cu") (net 8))
 (segment (start 67.785 163.9) (end 68.241 163.555) (width 0.3048) (layer "B.Cu") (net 8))
 (segment (start 51.275 163.265) (end 51.275 109.925) (width 0.3048) (layer "B.Cu") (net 8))
 (segment (start 53.815 107.385) (end 53.815 107.131) (width 0.3048) (layer "B.Cu") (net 8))
 (segment (start 63.34 165.17) (end 66.515 165.17) (width 0.3048) (layer "B.Cu") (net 8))
 (segment (start 61.435 163.265) (end 61.741 163.555) (width 0.3048) (layer "B.Cu") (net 8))
 (segment (start 55.72 64.84) (end 53.18 64.84) (width 0.3048) (layer "B.Cu") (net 4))
 (segment (start 56.355 114.37) (end 56.355 114.751) (width 0.3048) (layer "B.Cu") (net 4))
 (segment (start 60.165 110.56) (end 56.355 114.37) (width 0.3048) (layer "B.Cu") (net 4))
 (segment (start 53.18 64.84) (end 53.18 68.65) (width 0.3048) (layer "B.Cu") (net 4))
 (segment (start 77.945 95.32) (end 62.705 110.56) (width 0.3048) (layer "B.Cu") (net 4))
 (segment (start 53.18 68.65) (end 57.625 73.095) (width 0.3048) (layer "B.Cu") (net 4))
 (segment (start 62.705 110.56) (end 60.165 110.56) (width 0.3048) (layer "B.Cu") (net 4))
 (segment (start 57.625 73.095) (end 77.945 73.095) (width 0.3048) (layer "B.Cu") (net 4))
 (segment (start 77.945 73.095) (end 77.945 95.32) (width 0.3048) (layer "B.Cu") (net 4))
 (segment (start 50.64 88.335) (end 51.275 88.97) (width 0.3048) (layer "F.Cu") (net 7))
 (segment (start 60.8 76.27) (end 65.245 76.27) (width 0.3048) (layer "F.Cu") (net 7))
 (segment (start 65.245 76.27) (end 65.499 76.463) (width 0.3048) (layer "F.Cu") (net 7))
 (segment (start 51.275 84.525) (end 50.64 85.16) (width 0.3048) (layer "F.Cu") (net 7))
 (segment (start 60.8 76.905) (end 60.875 77.195) (width 0.3048) (layer "F.Cu") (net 7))
 (segment (start 50.64 85.16) (end 50.64 88.335) (width 0.3048) (layer "F.Cu") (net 7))
 (segment (start 60.8 76.905) (end 60.8 76.27) (width 0.3048) (layer "F.Cu") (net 7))
 (segment (start 51.275 79.445) (end 51.275 84.525) (width 0.3048) (layer "F.Cu") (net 7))
 (segment (start 53.815 76.905) (end 54.375 77.195) (width 0.3048) (layer "F.Cu") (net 7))
 (segment (start 51.275 109.29) (end 53.815 111.83) (width 0.3048) (layer "F.Cu") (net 7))
 (segment (start 53.815 76.905) (end 51.275 79.445) (width 0.3048) (layer "F.Cu") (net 7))
 (segment (start 51.275 88.97) (end 51.275 109.29) (width 0.3048) (layer "F.Cu") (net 7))
 (segment (start 53.815 111.83) (end 53.815 112.211) (width 0.3048) (layer "F.Cu") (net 7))
 (segment (start 56.99 78.81) (end 59.53 78.81) (width 0.3048) (layer "B.Cu") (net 7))
 (segment (start 59.53 78.81) (end 60.8 77.54) (width 0.3048) (layer "B.Cu") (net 7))
 (segment (start 54.45 77.54) (end 54.375 77.195) (width 0.3048) (layer "B.Cu") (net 7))
 (segment (start 55.72 77.54) (end 56.99 78.81) (width 0.3048) (layer "B.Cu") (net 7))
 (segment (start 60.8 77.54) (end 60.875 77.195) (width 0.3048) (layer "B.Cu") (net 7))
 (segment (start 54.45 77.54) (end 55.72 77.54) (width 0.3048) (layer "B.Cu") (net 7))
 (segment (start 64.61 163.265) (end 64.61 165.805) (width 0.3048) (layer "F.Cu") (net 10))
 (segment (start 64.61 165.805) (end 56.035 165.805) (width 0.3048) (layer "F.Cu") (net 10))
 (segment (start 64.61 163.265) (end 64.991 163.105) (width 0.3048) (layer "F.Cu") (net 10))
 (segment (start 74.135 81.35) (end 74.135 87.065) (width 0.3048) (layer "F.Cu") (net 9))
 (segment (start 72.865 80.08) (end 74.135 81.35) (width 0.3048) (layer "F.Cu") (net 9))
 (segment (start 72.865 76.905) (end 72.357 76.745) (width 0.3048) (layer "F.Cu") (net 9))
 (segment (start 72.865 76.905) (end 72.865 80.08) (width 0.3048) (layer "F.Cu") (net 9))
 (segment (start 74.135 87.065) (end 74.455 87.319) (width 0.3048) (layer "F.Cu") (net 9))
 (segment (start 51.91 86.43) (end 52.103 86.811) (width 0.3048) (layer "F.Cu") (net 5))
 (segment (start 57.625 76.745) (end 57.625 78.81) (width 0.3048) (layer "F.Cu") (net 5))
 (segment (start 51.91 80.715) (end 51.91 86.43) (width 0.3048) (layer "F.Cu") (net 5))
 (segment (start 57.625 78.81) (end 53.815 78.81) (width 0.3048) (layer "F.Cu") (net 5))
 (segment (start 53.815 78.81) (end 51.91 80.715) (width 0.3048) (layer "F.Cu") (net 5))
 (segment (start 66.515 86.43) (end 66.7309 85.847218) (width 0.3048) (layer "F.Cu") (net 3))
 (segment (start 60.8 115.64) (end 56.99 119.45) (width 0.3048) (layer "F.Cu") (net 3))
 (segment (start 66.515 86.43) (end 66.515 88.335) (width 0.3048) (layer "F.Cu") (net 3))
 (segment (start 60.8 94.05) (end 60.8 115.64) (width 0.3048) (layer "F.Cu") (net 3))
 (segment (start 66.515 88.335) (end 60.8 94.05) (width 0.3048) (layer "F.Cu") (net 3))
 (via (at 56.99 119.45) (size 1.2192) (drill 0.6096) (layers "F.Cu" "B.Cu") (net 3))
 (segment (start 55.72 119.45) (end 53.815 117.545) (width 0.3048) (layer "B.Cu") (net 3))
 (segment (start 56.99 119.45) (end 55.72 119.45) (width 0.3048) (layer "B.Cu") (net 3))
 (segment (start 53.815 117.545) (end 53.815 117.291) (width 0.3048) (layer "B.Cu") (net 3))
 (segment (start 71.595 99.765) (end 72.23 99.765) (width 0.3048) (layer "B.Cu") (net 14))
 (segment (start 56.355 109.925) (end 56.355 109.671) (width 0.3048) (layer "B.Cu") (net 14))
 (segment (start 72.23 82.62) (end 72.357 82.145) (width 0.3048) (layer "B.Cu") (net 14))
 (segment (start 72.23 99.765) (end 72.23 82.62) (width 0.3048) (layer "B.Cu") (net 14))
 (segment (start 56.355 109.925) (end 61.435 109.925) (width 0.3048) (layer "B.Cu") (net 14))
 (segment (start 61.435 109.925) (end 71.595 99.765) (width 0.3048) (layer "B.Cu") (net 14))
 (segment (start 69.055 160.725) (end 65.88 163.9) (width 0.3048) (layer "F.Cu") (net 11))
 (segment (start 65.245 168.345) (end 64.991 168.505) (width 0.3048) (layer "F.Cu") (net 11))
 (segment (start 65.88 163.9) (end 65.88 167.71) (width 0.3048) (layer "F.Cu") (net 11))
 (segment (start 62.07 107.385) (end 62.07 150.565) (width 0.3048) (layer "F.Cu") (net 11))
 (segment (start 62.07 150.565) (end 69.055 157.55) (width 0.3048) (layer "F.Cu") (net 11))
 (segment (start 69.055 157.55) (end 69.055 160.725) (width 0.3048) (layer "F.Cu") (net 11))
 (segment (start 65.88 167.71) (end 65.245 168.345) (width 0.3048) (layer "F.Cu") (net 11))
 (via (at 62.07 107.385) (size 1.2192) (drill 0.6096) (layers "F.Cu" "B.Cu") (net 11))
 (segment (start 56.355 107.385) (end 56.355 107.131) (width 0.3048) (layer "B.Cu") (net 11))
 (segment (start 56.355 107.385) (end 62.07 107.385) (width 0.3048) (layer "B.Cu") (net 11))
 (segment (start 58.895 109.925) (end 58.895 94.685) (width 0.3048) (layer "F.Cu") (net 6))
 (segment (start 58.895 94.685) (end 56.99 92.78) (width 0.3048) (layer "F.Cu") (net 6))
 (segment (start 56.355 112.465) (end 56.355 112.211) (width 0.3048) (layer "F.Cu") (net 6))
 (segment (start 56.355 112.465) (end 58.895 109.925) (width 0.3048) (layer "F.Cu") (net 6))
 (via (at 56.99 92.78) (size 1.2192) (drill 0.6096) (layers "F.Cu" "B.Cu") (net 6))
 (segment (start 56.99 92.78) (end 57.625 92.78) (width 0.3048) (layer "B.Cu") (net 6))
 (segment (start 57.625 92.78) (end 57.625 82.145) (width 0.3048) (layer "B.Cu") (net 6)))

